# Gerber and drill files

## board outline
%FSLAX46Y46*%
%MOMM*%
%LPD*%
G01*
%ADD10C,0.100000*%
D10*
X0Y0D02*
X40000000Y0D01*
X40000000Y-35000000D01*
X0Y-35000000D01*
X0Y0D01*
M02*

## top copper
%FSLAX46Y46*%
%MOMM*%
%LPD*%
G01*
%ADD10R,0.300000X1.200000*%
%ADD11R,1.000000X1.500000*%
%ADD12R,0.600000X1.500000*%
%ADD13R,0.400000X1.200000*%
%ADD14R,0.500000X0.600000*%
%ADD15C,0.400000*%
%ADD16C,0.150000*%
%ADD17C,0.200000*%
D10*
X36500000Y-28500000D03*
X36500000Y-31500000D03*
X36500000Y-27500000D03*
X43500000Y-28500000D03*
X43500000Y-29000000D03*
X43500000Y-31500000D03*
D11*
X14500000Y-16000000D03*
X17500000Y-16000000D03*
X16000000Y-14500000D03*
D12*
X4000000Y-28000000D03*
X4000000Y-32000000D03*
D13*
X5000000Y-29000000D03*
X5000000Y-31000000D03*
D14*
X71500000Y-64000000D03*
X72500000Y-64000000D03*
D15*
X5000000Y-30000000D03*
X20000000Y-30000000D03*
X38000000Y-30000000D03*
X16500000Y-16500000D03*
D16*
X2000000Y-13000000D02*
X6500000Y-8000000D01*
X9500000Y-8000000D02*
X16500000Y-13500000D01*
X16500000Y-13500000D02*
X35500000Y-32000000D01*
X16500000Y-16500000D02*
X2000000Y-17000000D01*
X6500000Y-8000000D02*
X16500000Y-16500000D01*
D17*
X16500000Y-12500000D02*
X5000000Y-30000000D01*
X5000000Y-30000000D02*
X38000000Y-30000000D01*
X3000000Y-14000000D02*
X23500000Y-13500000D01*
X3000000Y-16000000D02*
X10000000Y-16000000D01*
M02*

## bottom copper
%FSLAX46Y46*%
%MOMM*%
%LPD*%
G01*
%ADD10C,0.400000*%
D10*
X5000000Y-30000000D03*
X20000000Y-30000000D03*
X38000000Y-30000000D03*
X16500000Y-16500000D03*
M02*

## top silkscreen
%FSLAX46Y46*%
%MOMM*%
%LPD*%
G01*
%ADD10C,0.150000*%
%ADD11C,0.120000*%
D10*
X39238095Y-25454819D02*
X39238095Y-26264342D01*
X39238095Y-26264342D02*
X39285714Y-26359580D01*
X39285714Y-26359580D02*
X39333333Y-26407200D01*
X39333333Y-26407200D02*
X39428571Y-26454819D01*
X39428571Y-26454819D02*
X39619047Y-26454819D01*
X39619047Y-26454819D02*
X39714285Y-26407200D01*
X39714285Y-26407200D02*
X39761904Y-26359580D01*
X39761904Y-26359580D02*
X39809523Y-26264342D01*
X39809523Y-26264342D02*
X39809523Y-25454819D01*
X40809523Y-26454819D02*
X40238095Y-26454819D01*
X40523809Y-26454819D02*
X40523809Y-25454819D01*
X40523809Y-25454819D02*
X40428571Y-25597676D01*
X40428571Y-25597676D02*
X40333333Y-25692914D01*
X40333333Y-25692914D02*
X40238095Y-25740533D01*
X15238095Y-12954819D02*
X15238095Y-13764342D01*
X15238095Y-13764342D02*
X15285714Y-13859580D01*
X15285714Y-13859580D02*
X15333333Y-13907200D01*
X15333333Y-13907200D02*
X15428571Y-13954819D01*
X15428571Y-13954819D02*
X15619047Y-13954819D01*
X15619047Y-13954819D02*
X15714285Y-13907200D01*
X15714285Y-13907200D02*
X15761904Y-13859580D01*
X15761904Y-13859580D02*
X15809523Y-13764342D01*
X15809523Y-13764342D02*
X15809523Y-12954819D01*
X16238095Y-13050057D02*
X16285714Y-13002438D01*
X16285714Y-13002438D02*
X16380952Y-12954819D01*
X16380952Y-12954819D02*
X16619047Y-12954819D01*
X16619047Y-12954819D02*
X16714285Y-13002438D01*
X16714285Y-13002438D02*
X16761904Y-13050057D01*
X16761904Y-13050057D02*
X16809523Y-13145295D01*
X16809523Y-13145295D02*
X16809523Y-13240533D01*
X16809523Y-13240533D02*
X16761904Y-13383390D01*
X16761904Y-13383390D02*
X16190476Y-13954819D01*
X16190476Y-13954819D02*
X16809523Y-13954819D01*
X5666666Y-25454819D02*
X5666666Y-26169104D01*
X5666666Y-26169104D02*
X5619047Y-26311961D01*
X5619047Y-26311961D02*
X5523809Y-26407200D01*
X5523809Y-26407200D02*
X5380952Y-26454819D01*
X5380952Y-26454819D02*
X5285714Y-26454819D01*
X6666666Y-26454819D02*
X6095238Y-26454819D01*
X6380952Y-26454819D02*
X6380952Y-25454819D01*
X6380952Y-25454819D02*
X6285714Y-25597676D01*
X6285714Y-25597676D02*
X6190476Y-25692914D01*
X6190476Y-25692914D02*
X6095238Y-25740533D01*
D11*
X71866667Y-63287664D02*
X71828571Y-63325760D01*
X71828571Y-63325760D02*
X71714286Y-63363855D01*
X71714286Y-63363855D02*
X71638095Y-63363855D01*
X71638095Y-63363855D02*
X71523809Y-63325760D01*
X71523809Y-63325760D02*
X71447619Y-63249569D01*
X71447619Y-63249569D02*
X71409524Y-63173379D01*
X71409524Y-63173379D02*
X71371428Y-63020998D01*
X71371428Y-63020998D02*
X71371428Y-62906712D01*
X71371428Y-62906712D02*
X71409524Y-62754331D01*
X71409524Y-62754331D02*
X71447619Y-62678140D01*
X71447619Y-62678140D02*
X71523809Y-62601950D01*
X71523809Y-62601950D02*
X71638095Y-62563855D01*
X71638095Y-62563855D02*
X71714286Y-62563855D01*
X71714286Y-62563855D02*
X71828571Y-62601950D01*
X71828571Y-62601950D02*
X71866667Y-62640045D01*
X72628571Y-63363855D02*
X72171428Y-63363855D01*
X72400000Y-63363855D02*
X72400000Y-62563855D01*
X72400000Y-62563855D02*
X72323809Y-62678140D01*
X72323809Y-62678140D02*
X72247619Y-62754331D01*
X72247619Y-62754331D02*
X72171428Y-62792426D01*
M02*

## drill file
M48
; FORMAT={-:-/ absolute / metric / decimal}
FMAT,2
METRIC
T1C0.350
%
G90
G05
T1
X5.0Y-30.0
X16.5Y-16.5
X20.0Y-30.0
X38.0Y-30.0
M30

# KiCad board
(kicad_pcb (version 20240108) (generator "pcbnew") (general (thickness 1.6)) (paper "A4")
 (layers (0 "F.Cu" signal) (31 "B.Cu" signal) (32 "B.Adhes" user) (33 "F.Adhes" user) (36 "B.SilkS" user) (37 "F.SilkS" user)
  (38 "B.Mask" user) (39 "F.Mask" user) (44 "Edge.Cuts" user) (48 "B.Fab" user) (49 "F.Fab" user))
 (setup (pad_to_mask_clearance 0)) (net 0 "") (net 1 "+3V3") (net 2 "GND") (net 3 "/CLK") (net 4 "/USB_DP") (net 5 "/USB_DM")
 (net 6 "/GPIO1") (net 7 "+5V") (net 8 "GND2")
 (gr_rect (start 0 0) (end 40 35) (layer "Edge.Cuts") (width 0.1))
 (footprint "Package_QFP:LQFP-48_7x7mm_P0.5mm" (layer "F.Cu") (at 20 15 0)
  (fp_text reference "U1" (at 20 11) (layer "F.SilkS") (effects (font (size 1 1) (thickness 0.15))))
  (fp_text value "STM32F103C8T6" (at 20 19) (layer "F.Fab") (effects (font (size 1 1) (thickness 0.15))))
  (pad "8" smd rect (at 16.5 13.5) (size 0.3 1.2) (layers "F.Cu" "F.Paste" "F.Mask") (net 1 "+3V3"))
  (pad "23" smd rect (at 16.5 16.5) (size 0.3 1.2) (layers "F.Cu" "F.Paste" "F.Mask") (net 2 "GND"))
  (pad "5" smd rect (at 16.5 12.5) (size 0.3 1.2) (layers "F.Cu" "F.Paste" "F.Mask") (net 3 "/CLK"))
  (pad "44" smd rect (at 23.5 13.5) (size 0.3 1.2) (layers "F.Cu" "F.Paste" "F.Mask") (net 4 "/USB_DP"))
  (pad "43" smd rect (at 23.5 14.0) (size 0.3 1.2) (layers "F.Cu" "F.Paste" "F.Mask") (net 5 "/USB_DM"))
  (pad "20" smd rect (at 23.5 16.5) (size 0.3 1.2) (layers "F.Cu" "F.Paste" "F.Mask") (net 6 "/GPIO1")))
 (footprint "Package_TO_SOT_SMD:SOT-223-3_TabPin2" (layer "F.Cu") (at 8 8 0)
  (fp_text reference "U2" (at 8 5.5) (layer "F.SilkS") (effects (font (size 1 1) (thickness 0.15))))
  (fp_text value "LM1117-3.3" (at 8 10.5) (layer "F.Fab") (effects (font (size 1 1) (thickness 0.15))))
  (pad "1" smd rect (at 6.5 8) (size 1 1.5) (layers "F.Cu" "F.Paste" "F.Mask") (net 2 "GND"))
  (pad "2" smd rect (at 9.5 8) (size 1 1.5) (layers "F.Cu" "F.Paste" "F.Mask") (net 1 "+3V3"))
  (pad "3" smd rect (at 8 6.5) (size 1 1.5) (layers "F.Cu" "F.Paste" "F.Mask") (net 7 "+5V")))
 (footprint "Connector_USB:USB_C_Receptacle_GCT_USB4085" (layer "F.Cu") (at 2 15 0)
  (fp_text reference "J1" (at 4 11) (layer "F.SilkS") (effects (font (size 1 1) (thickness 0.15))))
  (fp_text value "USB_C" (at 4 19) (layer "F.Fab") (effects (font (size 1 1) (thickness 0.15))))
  (pad "VBUS" smd rect (at 2 13) (size 0.6 1.5) (layers "F.Cu" "F.Paste" "F.Mask") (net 7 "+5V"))
  (pad "GND" smd rect (at 2 17) (size 0.6 1.5) (layers "F.Cu" "F.Paste" "F.Mask") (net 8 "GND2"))
  (pad "DP" smd rect (at 3 14) (size 0.4 1.2) (layers "F.Cu" "F.Paste" "F.Mask") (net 4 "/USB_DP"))
  (pad "DM" smd rect (at 3 16) (size 0.4 1.2) (layers "F.Cu" "F.Paste" "F.Mask") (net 5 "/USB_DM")))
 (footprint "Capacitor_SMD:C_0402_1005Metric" (layer "F.Cu") (at 36 32 0)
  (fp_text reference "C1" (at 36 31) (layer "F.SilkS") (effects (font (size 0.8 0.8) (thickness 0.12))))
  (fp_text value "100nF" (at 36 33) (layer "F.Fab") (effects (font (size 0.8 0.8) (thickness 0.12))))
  (pad "1" smd rect (at 35.5 32) (size 0.5 0.6) (layers "F.Cu" "F.Paste" "F.Mask") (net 1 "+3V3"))
  (pad "2" smd rect (at 36.5 32) (size 0.5 0.6) (layers "F.Cu" "F.Paste" "F.Mask") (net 2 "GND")))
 (segment (start 2 13) (end 6.5 8) (width 0.15) (layer "F.Cu") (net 7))
 (segment (start 9.5 8) (end 16.5 13.5) (width 0.15) (layer "F.Cu") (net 1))
 (segment (start 16.5 13.5) (end 35.5 32) (width 0.15) (layer "F.Cu") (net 1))
 (segment (start 16.5 16.5) (end 2 17) (width 0.15) (layer "F.Cu") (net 2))
 (segment (start 6.5 8) (end 16.5 16.5) (width 0.15) (layer "F.Cu") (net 2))
 (segment (start 16.5 12.5) (end 5 30) (width 0.2) (layer "F.Cu") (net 3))
 (segment (start 5 30) (end 38 30) (width 0.2) (layer "F.Cu") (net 3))
 (segment (start 3 14) (end 23.5 13.5) (width 0.2) (layer "F.Cu") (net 4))
 (segment (start 3 16) (end 10 16) (width 0.2) (layer "F.Cu") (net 5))
 (via (at 5 30) (size 0.4) (drill 0.35) (layers "F.Cu" "B.Cu") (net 3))
 (via (at 20 30) (size 0.4) (drill 0.35) (layers "F.Cu" "B.Cu") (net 3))
 (via (at 38 30) (size 0.4) (drill 0.35) (layers "F.Cu" "B.Cu") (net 3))
 (via (at 16.5 16.5) (size 0.4) (drill 0.35) (layers "F.Cu" "B.Cu") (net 2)))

